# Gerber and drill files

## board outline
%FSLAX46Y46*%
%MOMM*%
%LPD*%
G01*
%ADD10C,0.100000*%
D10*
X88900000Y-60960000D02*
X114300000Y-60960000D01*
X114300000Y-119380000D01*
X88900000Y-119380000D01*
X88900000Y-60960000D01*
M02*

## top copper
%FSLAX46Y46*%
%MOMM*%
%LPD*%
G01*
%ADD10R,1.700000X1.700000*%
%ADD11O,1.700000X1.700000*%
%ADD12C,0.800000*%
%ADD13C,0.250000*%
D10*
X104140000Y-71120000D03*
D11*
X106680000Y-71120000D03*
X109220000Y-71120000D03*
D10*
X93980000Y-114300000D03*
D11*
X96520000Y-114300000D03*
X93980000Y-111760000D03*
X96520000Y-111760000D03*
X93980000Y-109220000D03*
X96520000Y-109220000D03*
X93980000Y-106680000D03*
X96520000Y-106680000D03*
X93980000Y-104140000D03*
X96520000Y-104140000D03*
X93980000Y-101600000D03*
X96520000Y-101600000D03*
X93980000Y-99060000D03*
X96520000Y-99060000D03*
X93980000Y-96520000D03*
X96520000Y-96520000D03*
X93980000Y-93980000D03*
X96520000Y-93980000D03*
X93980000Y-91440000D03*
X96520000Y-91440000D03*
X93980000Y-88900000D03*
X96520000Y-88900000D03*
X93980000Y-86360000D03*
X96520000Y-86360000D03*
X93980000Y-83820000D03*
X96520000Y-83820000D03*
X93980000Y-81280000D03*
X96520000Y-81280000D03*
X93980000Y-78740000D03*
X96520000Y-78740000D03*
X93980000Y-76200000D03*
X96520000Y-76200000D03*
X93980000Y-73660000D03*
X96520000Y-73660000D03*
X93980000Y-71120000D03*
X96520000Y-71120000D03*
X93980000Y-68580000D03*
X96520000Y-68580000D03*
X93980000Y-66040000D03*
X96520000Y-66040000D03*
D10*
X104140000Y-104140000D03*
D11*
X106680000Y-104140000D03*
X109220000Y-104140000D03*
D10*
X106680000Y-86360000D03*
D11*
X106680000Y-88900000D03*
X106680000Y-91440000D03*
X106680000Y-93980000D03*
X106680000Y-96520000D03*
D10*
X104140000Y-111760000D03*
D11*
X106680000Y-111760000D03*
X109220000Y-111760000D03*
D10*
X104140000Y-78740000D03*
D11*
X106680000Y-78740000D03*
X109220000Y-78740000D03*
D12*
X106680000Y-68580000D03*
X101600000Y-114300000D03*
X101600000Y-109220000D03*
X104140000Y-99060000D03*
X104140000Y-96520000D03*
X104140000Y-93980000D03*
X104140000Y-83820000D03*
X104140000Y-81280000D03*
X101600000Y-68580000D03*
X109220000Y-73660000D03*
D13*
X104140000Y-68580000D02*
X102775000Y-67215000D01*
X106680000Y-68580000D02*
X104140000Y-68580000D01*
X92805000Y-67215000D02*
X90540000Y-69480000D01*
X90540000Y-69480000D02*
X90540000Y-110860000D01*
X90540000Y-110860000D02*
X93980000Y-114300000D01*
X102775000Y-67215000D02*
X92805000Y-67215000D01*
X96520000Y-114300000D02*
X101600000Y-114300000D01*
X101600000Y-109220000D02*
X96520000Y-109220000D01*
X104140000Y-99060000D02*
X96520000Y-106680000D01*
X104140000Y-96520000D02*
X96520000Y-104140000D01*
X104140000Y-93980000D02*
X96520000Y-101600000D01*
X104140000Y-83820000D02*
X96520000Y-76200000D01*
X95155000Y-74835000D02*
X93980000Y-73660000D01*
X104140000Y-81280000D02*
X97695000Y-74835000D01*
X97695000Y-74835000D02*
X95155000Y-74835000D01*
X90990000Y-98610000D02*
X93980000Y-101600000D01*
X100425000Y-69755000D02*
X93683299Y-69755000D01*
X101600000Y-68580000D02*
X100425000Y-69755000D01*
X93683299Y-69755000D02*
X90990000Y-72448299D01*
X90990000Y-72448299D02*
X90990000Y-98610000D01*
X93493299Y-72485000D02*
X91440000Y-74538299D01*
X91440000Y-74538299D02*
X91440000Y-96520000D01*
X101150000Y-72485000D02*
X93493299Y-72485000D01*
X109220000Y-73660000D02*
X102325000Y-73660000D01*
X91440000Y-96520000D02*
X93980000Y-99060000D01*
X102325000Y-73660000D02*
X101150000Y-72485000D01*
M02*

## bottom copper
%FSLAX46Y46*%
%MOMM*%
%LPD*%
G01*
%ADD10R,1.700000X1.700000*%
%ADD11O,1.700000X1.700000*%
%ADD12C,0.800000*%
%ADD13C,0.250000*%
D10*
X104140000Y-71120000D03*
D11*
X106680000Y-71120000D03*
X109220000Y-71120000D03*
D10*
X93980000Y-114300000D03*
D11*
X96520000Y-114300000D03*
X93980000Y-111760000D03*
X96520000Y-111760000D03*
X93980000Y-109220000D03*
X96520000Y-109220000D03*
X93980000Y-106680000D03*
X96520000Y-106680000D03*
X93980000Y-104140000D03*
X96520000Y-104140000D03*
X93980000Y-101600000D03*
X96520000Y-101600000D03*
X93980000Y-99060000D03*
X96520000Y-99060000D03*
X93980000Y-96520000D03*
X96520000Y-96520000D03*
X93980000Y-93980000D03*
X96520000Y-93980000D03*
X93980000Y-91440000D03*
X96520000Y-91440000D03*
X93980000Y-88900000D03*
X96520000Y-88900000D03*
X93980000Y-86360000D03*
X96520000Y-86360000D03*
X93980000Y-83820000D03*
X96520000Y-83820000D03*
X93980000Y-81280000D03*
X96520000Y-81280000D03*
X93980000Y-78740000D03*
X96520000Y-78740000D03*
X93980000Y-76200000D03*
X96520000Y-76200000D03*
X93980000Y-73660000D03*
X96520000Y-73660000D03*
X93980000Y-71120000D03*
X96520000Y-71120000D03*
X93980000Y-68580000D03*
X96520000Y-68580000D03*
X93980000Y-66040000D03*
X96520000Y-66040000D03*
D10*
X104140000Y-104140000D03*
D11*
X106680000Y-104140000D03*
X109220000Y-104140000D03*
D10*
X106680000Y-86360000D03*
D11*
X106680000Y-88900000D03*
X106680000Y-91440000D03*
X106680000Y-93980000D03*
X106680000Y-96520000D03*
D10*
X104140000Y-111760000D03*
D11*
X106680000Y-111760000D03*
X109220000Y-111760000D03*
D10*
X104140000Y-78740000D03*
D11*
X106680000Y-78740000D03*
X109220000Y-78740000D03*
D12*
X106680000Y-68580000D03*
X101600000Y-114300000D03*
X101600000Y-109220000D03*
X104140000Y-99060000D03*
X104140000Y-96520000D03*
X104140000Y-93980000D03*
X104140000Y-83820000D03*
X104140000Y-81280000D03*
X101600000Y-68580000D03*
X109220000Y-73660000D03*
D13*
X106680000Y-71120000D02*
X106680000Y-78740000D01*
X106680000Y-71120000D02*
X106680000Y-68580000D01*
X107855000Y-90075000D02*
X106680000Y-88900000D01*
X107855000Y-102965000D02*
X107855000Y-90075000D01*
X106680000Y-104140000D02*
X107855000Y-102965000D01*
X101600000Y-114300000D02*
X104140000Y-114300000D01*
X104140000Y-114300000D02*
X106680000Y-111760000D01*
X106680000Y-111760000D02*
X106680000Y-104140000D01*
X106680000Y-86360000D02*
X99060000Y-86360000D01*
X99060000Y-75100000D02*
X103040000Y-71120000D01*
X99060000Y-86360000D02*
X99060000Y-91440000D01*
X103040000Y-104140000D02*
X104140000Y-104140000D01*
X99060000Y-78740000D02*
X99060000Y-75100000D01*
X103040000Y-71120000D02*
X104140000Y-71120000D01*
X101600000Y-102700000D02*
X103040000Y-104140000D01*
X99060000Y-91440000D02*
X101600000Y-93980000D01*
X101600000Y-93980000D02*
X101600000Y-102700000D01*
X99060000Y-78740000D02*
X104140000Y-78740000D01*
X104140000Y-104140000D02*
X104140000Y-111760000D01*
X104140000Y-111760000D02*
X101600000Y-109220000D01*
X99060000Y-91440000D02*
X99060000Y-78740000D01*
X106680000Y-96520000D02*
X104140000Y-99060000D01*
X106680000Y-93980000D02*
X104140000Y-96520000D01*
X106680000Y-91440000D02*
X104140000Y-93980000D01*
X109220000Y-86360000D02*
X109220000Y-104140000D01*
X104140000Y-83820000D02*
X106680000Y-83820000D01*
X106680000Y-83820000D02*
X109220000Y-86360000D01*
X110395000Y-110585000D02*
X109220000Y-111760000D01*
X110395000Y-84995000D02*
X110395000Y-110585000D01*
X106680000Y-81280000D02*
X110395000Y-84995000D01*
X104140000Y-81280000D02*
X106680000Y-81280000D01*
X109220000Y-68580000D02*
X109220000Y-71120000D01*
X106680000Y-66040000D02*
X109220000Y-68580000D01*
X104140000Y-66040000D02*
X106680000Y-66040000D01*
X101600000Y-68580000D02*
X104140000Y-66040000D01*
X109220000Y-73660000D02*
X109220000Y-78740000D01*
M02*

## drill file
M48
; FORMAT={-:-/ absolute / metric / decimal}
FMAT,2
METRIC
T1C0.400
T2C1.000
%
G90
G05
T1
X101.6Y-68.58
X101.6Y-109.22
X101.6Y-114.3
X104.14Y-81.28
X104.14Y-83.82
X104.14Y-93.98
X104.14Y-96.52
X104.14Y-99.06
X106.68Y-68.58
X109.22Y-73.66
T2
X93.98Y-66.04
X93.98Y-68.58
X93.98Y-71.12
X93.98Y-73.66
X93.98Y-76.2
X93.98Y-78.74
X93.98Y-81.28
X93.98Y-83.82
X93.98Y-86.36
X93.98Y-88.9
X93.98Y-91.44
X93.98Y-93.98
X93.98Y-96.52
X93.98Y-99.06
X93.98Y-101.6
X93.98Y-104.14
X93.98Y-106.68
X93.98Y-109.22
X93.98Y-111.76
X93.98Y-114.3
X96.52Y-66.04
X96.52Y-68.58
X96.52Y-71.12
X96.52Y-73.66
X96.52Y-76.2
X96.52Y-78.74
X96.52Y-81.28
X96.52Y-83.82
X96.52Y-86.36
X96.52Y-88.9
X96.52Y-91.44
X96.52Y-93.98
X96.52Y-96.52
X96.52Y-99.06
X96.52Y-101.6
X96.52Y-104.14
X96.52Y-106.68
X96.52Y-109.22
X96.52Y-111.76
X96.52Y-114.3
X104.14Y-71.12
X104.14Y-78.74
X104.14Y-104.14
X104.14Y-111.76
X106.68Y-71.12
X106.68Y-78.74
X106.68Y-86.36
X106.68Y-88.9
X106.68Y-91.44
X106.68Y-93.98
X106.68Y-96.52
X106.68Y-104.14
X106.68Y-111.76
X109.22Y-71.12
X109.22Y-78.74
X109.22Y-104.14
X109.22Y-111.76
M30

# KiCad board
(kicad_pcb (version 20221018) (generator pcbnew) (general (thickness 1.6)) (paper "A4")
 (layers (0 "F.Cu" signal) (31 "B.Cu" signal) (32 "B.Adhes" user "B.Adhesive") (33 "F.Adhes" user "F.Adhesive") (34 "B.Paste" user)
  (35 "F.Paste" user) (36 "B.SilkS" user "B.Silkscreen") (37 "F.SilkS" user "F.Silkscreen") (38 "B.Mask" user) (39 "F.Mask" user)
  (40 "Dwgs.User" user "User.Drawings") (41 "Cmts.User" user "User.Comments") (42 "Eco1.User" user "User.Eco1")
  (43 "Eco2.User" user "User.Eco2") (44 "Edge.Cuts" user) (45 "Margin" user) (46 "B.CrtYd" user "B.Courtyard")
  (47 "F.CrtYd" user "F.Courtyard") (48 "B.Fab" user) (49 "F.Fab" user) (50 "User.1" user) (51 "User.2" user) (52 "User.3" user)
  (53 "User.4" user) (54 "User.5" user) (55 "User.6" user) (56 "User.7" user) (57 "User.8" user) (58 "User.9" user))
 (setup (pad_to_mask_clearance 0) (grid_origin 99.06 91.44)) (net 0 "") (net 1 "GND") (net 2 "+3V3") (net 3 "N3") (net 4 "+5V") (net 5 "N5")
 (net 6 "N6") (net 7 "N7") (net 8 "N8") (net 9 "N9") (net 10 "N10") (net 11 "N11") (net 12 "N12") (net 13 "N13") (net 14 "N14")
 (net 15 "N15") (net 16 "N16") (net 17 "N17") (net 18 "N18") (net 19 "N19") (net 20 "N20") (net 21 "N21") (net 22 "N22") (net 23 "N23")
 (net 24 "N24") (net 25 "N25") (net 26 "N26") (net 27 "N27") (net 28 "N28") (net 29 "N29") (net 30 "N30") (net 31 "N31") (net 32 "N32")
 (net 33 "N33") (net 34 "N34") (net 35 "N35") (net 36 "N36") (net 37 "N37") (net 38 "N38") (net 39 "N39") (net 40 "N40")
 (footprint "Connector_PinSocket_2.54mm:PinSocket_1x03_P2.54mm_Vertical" (layer "F.Cu") (at 104.14 71.12 90)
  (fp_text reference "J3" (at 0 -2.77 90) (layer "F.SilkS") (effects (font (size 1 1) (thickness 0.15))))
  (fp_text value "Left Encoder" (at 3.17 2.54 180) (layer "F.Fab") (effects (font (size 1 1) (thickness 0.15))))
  (pad "1" thru_hole rect (at 0 0 90) (size 1.7 1.7) (drill 1) (layers "*.Cu" "*.Mask") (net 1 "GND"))
  (pad "2" thru_hole oval (at 0 2.54 90) (size 1.7 1.7) (drill 1) (layers "*.Cu" "*.Mask") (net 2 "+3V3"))
  (pad "3" thru_hole oval (at 0 5.08 90) (size 1.7 1.7) (drill 1) (layers "*.Cu" "*.Mask") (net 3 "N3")))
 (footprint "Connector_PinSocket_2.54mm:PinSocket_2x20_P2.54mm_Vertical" (layer "F.Cu") (at 93.98 114.3 180)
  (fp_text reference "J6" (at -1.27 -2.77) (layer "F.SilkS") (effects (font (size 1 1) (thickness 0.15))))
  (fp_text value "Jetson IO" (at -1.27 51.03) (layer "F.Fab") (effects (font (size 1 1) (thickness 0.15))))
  (pad "1" thru_hole rect (at 0 0 180) (size 1.7 1.7) (drill 1) (layers "*.Cu" "*.Mask") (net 2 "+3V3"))
  (pad "2" thru_hole oval (at -2.54 0 180) (size 1.7 1.7) (drill 1) (layers "*.Cu" "*.Mask") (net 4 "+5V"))
  (pad "3" thru_hole oval (at 0 2.54 180) (size 1.7 1.7) (drill 1) (layers "*.Cu" "*.Mask") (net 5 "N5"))
  (pad "4" thru_hole oval (at -2.54 2.54 180) (size 1.7 1.7) (drill 1) (layers "*.Cu" "*.Mask") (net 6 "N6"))
  (pad "5" thru_hole oval (at 0 5.08 180) (size 1.7 1.7) (drill 1) (layers "*.Cu" "*.Mask") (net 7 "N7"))
  (pad "6" thru_hole oval (at -2.54 5.08 180) (size 1.7 1.7) (drill 1) (layers "*.Cu" "*.Mask") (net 1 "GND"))
  (pad "7" thru_hole oval (at 0 7.62 180) (size 1.7 1.7) (drill 1) (layers "*.Cu" "*.Mask") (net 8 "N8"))
  (pad "8" thru_hole oval (at -2.54 7.62 180) (size 1.7 1.7) (drill 1) (layers "*.Cu" "*.Mask") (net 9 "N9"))
  (pad "9" thru_hole oval (at 0 10.16 180) (size 1.7 1.7) (drill 1) (layers "*.Cu" "*.Mask") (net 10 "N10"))
  (pad "10" thru_hole oval (at -2.54 10.16 180) (size 1.7 1.7) (drill 1) (layers "*.Cu" "*.Mask") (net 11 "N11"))
  (pad "11" thru_hole oval (at 0 12.7 180) (size 1.7 1.7) (drill 1) (layers "*.Cu" "*.Mask") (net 3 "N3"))
  (pad "12" thru_hole oval (at -2.54 12.7 180) (size 1.7 1.7) (drill 1) (layers "*.Cu" "*.Mask") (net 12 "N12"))
  (pad "13" thru_hole oval (at 0 15.24 180) (size 1.7 1.7) (drill 1) (layers "*.Cu" "*.Mask") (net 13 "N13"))
  (pad "14" thru_hole oval (at -2.54 15.24 180) (size 1.7 1.7) (drill 1) (layers "*.Cu" "*.Mask") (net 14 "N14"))
  (pad "15" thru_hole oval (at 0 17.78 180) (size 1.7 1.7) (drill 1) (layers "*.Cu" "*.Mask") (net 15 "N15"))
  (pad "16" thru_hole oval (at -2.54 17.78 180) (size 1.7 1.7) (drill 1) (layers "*.Cu" "*.Mask") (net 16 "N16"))
  (pad "17" thru_hole oval (at 0 20.32 180) (size 1.7 1.7) (drill 1) (layers "*.Cu" "*.Mask") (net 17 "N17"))
  (pad "18" thru_hole oval (at -2.54 20.32 180) (size 1.7 1.7) (drill 1) (layers "*.Cu" "*.Mask") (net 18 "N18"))
  (pad "19" thru_hole oval (at 0 22.86 180) (size 1.7 1.7) (drill 1) (layers "*.Cu" "*.Mask") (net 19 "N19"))
  (pad "20" thru_hole oval (at -2.54 22.86 180) (size 1.7 1.7) (drill 1) (layers "*.Cu" "*.Mask") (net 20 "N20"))
  (pad "21" thru_hole oval (at 0 25.4 180) (size 1.7 1.7) (drill 1) (layers "*.Cu" "*.Mask") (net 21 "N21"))
  (pad "22" thru_hole oval (at -2.54 25.4 180) (size 1.7 1.7) (drill 1) (layers "*.Cu" "*.Mask") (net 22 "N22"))
  (pad "23" thru_hole oval (at 0 27.94 180) (size 1.7 1.7) (drill 1) (layers "*.Cu" "*.Mask") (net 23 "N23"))
  (pad "24" thru_hole oval (at -2.54 27.94 180) (size 1.7 1.7) (drill 1) (layers "*.Cu" "*.Mask") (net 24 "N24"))
  (pad "25" thru_hole oval (at 0 30.48 180) (size 1.7 1.7) (drill 1) (layers "*.Cu" "*.Mask") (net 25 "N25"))
  (pad "26" thru_hole oval (at -2.54 30.48 180) (size 1.7 1.7) (drill 1) (layers "*.Cu" "*.Mask") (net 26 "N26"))
  (pad "27" thru_hole oval (at 0 33.02 180) (size 1.7 1.7) (drill 1) (layers "*.Cu" "*.Mask") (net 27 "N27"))
  (pad "28" thru_hole oval (at -2.54 33.02 180) (size 1.7 1.7) (drill 1) (layers "*.Cu" "*.Mask") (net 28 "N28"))
  (pad "29" thru_hole oval (at 0 35.56 180) (size 1.7 1.7) (drill 1) (layers "*.Cu" "*.Mask") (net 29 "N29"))
  (pad "30" thru_hole oval (at -2.54 35.56 180) (size 1.7 1.7) (drill 1) (layers "*.Cu" "*.Mask") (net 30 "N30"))
  (pad "31" thru_hole oval (at 0 38.1 180) (size 1.7 1.7) (drill 1) (layers "*.Cu" "*.Mask") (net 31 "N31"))
  (pad "32" thru_hole oval (at -2.54 38.1 180) (size 1.7 1.7) (drill 1) (layers "*.Cu" "*.Mask") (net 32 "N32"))
  (pad "33" thru_hole oval (at 0 40.64 180) (size 1.7 1.7) (drill 1) (layers "*.Cu" "*.Mask") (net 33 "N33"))
  (pad "34" thru_hole oval (at -2.54 40.64 180) (size 1.7 1.7) (drill 1) (layers "*.Cu" "*.Mask") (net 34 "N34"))
  (pad "35" thru_hole oval (at 0 43.18 180) (size 1.7 1.7) (drill 1) (layers "*.Cu" "*.Mask") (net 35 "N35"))
  (pad "36" thru_hole oval (at -2.54 43.18 180) (size 1.7 1.7) (drill 1) (layers "*.Cu" "*.Mask") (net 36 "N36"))
  (pad "37" thru_hole oval (at 0 45.72 180) (size 1.7 1.7) (drill 1) (layers "*.Cu" "*.Mask") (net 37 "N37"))
  (pad "38" thru_hole oval (at -2.54 45.72 180) (size 1.7 1.7) (drill 1) (layers "*.Cu" "*.Mask") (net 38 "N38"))
  (pad "39" thru_hole oval (at 0 48.26 180) (size 1.7 1.7) (drill 1) (layers "*.Cu" "*.Mask") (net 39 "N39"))
  (pad "40" thru_hole oval (at -2.54 48.26 180) (size 1.7 1.7) (drill 1) (layers "*.Cu" "*.Mask") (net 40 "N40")))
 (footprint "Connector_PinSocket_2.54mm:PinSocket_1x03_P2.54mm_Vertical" (layer "F.Cu") (at 104.14 104.14 90)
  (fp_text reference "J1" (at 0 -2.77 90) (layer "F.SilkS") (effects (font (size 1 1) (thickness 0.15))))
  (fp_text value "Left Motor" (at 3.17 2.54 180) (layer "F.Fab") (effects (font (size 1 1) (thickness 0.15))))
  (pad "1" thru_hole rect (at 0 0 90) (size 1.7 1.7) (drill 1) (layers "*.Cu" "*.Mask") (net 1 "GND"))
  (pad "2" thru_hole oval (at 0 2.54 90) (size 1.7 1.7) (drill 1) (layers "*.Cu" "*.Mask") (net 4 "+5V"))
  (pad "3" thru_hole oval (at 0 5.08 90) (size 1.7 1.7) (drill 1) (layers "*.Cu" "*.Mask") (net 32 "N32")))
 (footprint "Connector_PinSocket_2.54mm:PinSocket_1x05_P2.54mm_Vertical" (layer "F.Cu") (at 106.68 86.36)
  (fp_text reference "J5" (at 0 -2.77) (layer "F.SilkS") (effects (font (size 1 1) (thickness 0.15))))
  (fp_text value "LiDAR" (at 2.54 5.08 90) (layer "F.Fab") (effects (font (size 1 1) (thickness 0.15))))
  (pad "1" thru_hole rect (at 0 0) (size 1.7 1.7) (drill 1) (layers "*.Cu" "*.Mask") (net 1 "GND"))
  (pad "2" thru_hole oval (at 0 2.54) (size 1.7 1.7) (drill 1) (layers "*.Cu" "*.Mask") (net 4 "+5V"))
  (pad "3" thru_hole oval (at 0 5.08) (size 1.7 1.7) (drill 1) (layers "*.Cu" "*.Mask") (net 12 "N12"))
  (pad "4" thru_hole oval (at 0 7.62) (size 1.7 1.7) (drill 1) (layers "*.Cu" "*.Mask") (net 11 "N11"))
  (pad "5" thru_hole oval (at 0 10.16) (size 1.7 1.7) (drill 1) (layers "*.Cu" "*.Mask") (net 9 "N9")))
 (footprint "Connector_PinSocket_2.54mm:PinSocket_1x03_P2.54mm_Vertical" (layer "F.Cu") (at 104.14 111.76 90)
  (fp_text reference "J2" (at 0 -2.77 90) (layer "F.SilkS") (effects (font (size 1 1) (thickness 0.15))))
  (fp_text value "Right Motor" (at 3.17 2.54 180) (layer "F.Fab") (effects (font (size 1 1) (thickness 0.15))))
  (pad "1" thru_hole rect (at 0 0 90) (size 1.7 1.7) (drill 1) (layers "*.Cu" "*.Mask") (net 1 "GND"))
  (pad "2" thru_hole oval (at 0 2.54 90) (size 1.7 1.7) (drill 1) (layers "*.Cu" "*.Mask") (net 4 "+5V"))
  (pad "3" thru_hole oval (at 0 5.08 90) (size 1.7 1.7) (drill 1) (layers "*.Cu" "*.Mask") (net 33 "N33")))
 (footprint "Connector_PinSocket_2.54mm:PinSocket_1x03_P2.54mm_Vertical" (layer "F.Cu") (at 104.14 78.74 90)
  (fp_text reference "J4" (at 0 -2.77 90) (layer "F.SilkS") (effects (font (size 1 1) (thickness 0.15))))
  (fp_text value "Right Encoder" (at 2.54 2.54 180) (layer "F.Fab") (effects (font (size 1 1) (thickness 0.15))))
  (pad "1" thru_hole rect (at 0 0 90) (size 1.7 1.7) (drill 1) (layers "*.Cu" "*.Mask") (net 1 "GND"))
  (pad "2" thru_hole oval (at 0 2.54 90) (size 1.7 1.7) (drill 1) (layers "*.Cu" "*.Mask") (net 2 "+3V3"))
  (pad "3" thru_hole oval (at 0 5.08 90) (size 1.7 1.7) (drill 1) (layers "*.Cu" "*.Mask") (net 13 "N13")))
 (gr_rect (start 88.9 60.96) (end 114.3 119.38) (stroke (width 0.1) (type default)) (fill none) (layer "Edge.Cuts"))
 (segment (start 104.14 68.58) (end 102.775 67.215) (width 0.25) (layer "F.Cu") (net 2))
 (segment (start 106.68 68.58) (end 104.14 68.58) (width 0.25) (layer "F.Cu") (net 2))
 (segment (start 92.805 67.215) (end 90.54 69.48) (width 0.25) (layer "F.Cu") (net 2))
 (segment (start 90.54 69.48) (end 90.54 110.86) (width 0.25) (layer "F.Cu") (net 2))
 (segment (start 90.54 110.86) (end 93.98 114.3) (width 0.25) (layer "F.Cu") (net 2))
 (segment (start 102.775 67.215) (end 92.805 67.215) (width 0.25) (layer "F.Cu") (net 2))
 (via (at 106.68 68.58) (size 0.8) (drill 0.4) (layers "F.Cu" "B.Cu") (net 2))
 (segment (start 106.68 71.12) (end 106.68 78.74) (width 0.25) (layer "B.Cu") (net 2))
 (segment (start 106.68 71.12) (end 106.68 68.58) (width 0.25) (layer "B.Cu") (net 2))
 (segment (start 96.52 114.3) (end 101.6 114.3) (width 0.25) (layer "F.Cu") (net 4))
 (via (at 101.6 114.3) (size 0.8) (drill 0.4) (layers "F.Cu" "B.Cu") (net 4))
 (segment (start 107.855 90.075) (end 106.68 88.9) (width 0.25) (layer "B.Cu") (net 4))
 (segment (start 107.855 102.965) (end 107.855 90.075) (width 0.25) (layer "B.Cu") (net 4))
 (segment (start 106.68 104.14) (end 107.855 102.965) (width 0.25) (layer "B.Cu") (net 4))
 (segment (start 101.6 114.3) (end 104.14 114.3) (width 0.25) (layer "B.Cu") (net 4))
 (segment (start 104.14 114.3) (end 106.68 111.76) (width 0.25) (layer "B.Cu") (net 4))
 (segment (start 106.68 111.76) (end 106.68 104.14) (width 0.25) (layer "B.Cu") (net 4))
 (segment (start 101.6 109.22) (end 96.52 109.22) (width 0.25) (layer "F.Cu") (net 1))
 (via (at 101.6 109.22) (size 0.8) (drill 0.4) (layers "F.Cu" "B.Cu") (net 1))
 (segment (start 106.68 86.36) (end 99.06 86.36) (width 0.25) (layer "B.Cu") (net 1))
 (segment (start 99.06 75.1) (end 103.04 71.12) (width 0.25) (layer "B.Cu") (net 1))
 (segment (start 99.06 86.36) (end 99.06 91.44) (width 0.25) (layer "B.Cu") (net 1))
 (segment (start 103.04 104.14) (end 104.14 104.14) (width 0.25) (layer "B.Cu") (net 1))
 (segment (start 99.06 78.74) (end 99.06 75.1) (width 0.25) (layer "B.Cu") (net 1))
 (segment (start 103.04 71.12) (end 104.14 71.12) (width 0.25) (layer "B.Cu") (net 1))
 (segment (start 101.6 102.7) (end 103.04 104.14) (width 0.25) (layer "B.Cu") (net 1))
 (segment (start 99.06 91.44) (end 101.6 93.98) (width 0.25) (layer "B.Cu") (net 1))
 (segment (start 101.6 93.98) (end 101.6 102.7) (width 0.25) (layer "B.Cu") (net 1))
 (segment (start 99.06 78.74) (end 104.14 78.74) (width 0.25) (layer "B.Cu") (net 1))
 (segment (start 104.14 104.14) (end 104.14 111.76) (width 0.25) (layer "B.Cu") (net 1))
 (segment (start 104.14 111.76) (end 101.6 109.22) (width 0.25) (layer "B.Cu") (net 1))
 (segment (start 99.06 91.44) (end 99.06 78.74) (width 0.25) (layer "B.Cu") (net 1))
 (segment (start 104.14 99.06) (end 96.52 106.68) (width 0.25) (layer "F.Cu") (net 9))
 (via (at 104.14 99.06) (size 0.8) (drill 0.4) (layers "F.Cu" "B.Cu") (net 9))
 (segment (start 106.68 96.52) (end 104.14 99.06) (width 0.25) (layer "B.Cu") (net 9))
 (segment (start 104.14 96.52) (end 96.52 104.14) (width 0.25) (layer "F.Cu") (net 11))
 (via (at 104.14 96.52) (size 0.8) (drill 0.4) (layers "F.Cu" "B.Cu") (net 11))
 (segment (start 106.68 93.98) (end 104.14 96.52) (width 0.25) (layer "B.Cu") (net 11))
 (segment (start 104.14 93.98) (end 96.52 101.6) (width 0.25) (layer "F.Cu") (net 12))
 (via (at 104.14 93.98) (size 0.8) (drill 0.4) (layers "F.Cu" "B.Cu") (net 12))
 (segment (start 106.68 91.44) (end 104.14 93.98) (width 0.25) (layer "B.Cu") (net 12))
 (segment (start 104.14 83.82) (end 96.52 76.2) (width 0.25) (layer "F.Cu") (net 32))
 (via (at 104.14 83.82) (size 0.8) (drill 0.4) (layers "F.Cu" "B.Cu") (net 32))
 (segment (start 109.22 86.36) (end 109.22 104.14) (width 0.25) (layer "B.Cu") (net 32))
 (segment (start 104.14 83.82) (end 106.68 83.82) (width 0.25) (layer "B.Cu") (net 32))
 (segment (start 106.68 83.82) (end 109.22 86.36) (width 0.25) (layer "B.Cu") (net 32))
 (segment (start 95.155 74.835) (end 93.98 73.66) (width 0.25) (layer "F.Cu") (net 33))
 (segment (start 104.14 81.28) (end 97.695 74.835) (width 0.25) (layer "F.Cu") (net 33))
 (segment (start 97.695 74.835) (end 95.155 74.835) (width 0.25) (layer "F.Cu") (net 33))
 (via (at 104.14 81.28) (size 0.8) (drill 0.4) (layers "F.Cu" "B.Cu") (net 33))
 (segment (start 110.395 110.585) (end 109.22 111.76) (width 0.25) (layer "B.Cu") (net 33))
 (segment (start 110.395 84.995) (end 110.395 110.585) (width 0.25) (layer "B.Cu") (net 33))
 (segment (start 106.68 81.28) (end 110.395 84.995) (width 0.25) (layer "B.Cu") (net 33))
 (segment (start 104.14 81.28) (end 106.68 81.28) (width 0.25) (layer "B.Cu") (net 33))
 (segment (start 90.99 98.61) (end 93.98 101.6) (width 0.25) (layer "F.Cu") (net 3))
 (segment (start 100.425 69.755) (end 93.683299 69.755) (width 0.25) (layer "F.Cu") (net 3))
 (segment (start 101.6 68.58) (end 100.425 69.755) (width 0.25) (layer "F.Cu") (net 3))
 (segment (start 93.683299 69.755) (end 90.99 72.448299) (width 0.25) (layer "F.Cu") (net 3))
 (segment (start 90.99 72.448299) (end 90.99 98.61) (width 0.25) (layer "F.Cu") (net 3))
 (via (at 101.6 68.58) (size 0.8) (drill 0.4) (layers "F.Cu" "B.Cu") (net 3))
 (segment (start 109.22 68.58) (end 109.22 71.12) (width 0.25) (layer "B.Cu") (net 3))
 (segment (start 106.68 66.04) (end 109.22 68.58) (width 0.25) (layer "B.Cu") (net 3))
 (segment (start 104.14 66.04) (end 106.68 66.04) (width 0.25) (layer "B.Cu") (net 3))
 (segment (start 101.6 68.58) (end 104.14 66.04) (width 0.25) (layer "B.Cu") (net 3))
 (segment (start 93.493299 72.485) (end 91.44 74.538299) (width 0.25) (layer "F.Cu") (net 13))
 (segment (start 91.44 74.538299) (end 91.44 96.52) (width 0.25) (layer "F.Cu") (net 13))
 (segment (start 101.15 72.485) (end 93.493299 72.485) (width 0.25) (layer "F.Cu") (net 13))
 (segment (start 109.22 73.66) (end 102.325 73.66) (width 0.25) (layer "F.Cu") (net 13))
 (segment (start 91.44 96.52) (end 93.98 99.06) (width 0.25) (layer "F.Cu") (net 13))
 (segment (start 102.325 73.66) (end 101.15 72.485) (width 0.25) (layer "F.Cu") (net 13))
 (via (at 109.22 73.66) (size 0.8) (drill 0.4) (layers "F.Cu" "B.Cu") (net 13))
 (segment (start 109.22 73.66) (end 109.22 78.74) (width 0.25) (layer "B.Cu") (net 13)))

